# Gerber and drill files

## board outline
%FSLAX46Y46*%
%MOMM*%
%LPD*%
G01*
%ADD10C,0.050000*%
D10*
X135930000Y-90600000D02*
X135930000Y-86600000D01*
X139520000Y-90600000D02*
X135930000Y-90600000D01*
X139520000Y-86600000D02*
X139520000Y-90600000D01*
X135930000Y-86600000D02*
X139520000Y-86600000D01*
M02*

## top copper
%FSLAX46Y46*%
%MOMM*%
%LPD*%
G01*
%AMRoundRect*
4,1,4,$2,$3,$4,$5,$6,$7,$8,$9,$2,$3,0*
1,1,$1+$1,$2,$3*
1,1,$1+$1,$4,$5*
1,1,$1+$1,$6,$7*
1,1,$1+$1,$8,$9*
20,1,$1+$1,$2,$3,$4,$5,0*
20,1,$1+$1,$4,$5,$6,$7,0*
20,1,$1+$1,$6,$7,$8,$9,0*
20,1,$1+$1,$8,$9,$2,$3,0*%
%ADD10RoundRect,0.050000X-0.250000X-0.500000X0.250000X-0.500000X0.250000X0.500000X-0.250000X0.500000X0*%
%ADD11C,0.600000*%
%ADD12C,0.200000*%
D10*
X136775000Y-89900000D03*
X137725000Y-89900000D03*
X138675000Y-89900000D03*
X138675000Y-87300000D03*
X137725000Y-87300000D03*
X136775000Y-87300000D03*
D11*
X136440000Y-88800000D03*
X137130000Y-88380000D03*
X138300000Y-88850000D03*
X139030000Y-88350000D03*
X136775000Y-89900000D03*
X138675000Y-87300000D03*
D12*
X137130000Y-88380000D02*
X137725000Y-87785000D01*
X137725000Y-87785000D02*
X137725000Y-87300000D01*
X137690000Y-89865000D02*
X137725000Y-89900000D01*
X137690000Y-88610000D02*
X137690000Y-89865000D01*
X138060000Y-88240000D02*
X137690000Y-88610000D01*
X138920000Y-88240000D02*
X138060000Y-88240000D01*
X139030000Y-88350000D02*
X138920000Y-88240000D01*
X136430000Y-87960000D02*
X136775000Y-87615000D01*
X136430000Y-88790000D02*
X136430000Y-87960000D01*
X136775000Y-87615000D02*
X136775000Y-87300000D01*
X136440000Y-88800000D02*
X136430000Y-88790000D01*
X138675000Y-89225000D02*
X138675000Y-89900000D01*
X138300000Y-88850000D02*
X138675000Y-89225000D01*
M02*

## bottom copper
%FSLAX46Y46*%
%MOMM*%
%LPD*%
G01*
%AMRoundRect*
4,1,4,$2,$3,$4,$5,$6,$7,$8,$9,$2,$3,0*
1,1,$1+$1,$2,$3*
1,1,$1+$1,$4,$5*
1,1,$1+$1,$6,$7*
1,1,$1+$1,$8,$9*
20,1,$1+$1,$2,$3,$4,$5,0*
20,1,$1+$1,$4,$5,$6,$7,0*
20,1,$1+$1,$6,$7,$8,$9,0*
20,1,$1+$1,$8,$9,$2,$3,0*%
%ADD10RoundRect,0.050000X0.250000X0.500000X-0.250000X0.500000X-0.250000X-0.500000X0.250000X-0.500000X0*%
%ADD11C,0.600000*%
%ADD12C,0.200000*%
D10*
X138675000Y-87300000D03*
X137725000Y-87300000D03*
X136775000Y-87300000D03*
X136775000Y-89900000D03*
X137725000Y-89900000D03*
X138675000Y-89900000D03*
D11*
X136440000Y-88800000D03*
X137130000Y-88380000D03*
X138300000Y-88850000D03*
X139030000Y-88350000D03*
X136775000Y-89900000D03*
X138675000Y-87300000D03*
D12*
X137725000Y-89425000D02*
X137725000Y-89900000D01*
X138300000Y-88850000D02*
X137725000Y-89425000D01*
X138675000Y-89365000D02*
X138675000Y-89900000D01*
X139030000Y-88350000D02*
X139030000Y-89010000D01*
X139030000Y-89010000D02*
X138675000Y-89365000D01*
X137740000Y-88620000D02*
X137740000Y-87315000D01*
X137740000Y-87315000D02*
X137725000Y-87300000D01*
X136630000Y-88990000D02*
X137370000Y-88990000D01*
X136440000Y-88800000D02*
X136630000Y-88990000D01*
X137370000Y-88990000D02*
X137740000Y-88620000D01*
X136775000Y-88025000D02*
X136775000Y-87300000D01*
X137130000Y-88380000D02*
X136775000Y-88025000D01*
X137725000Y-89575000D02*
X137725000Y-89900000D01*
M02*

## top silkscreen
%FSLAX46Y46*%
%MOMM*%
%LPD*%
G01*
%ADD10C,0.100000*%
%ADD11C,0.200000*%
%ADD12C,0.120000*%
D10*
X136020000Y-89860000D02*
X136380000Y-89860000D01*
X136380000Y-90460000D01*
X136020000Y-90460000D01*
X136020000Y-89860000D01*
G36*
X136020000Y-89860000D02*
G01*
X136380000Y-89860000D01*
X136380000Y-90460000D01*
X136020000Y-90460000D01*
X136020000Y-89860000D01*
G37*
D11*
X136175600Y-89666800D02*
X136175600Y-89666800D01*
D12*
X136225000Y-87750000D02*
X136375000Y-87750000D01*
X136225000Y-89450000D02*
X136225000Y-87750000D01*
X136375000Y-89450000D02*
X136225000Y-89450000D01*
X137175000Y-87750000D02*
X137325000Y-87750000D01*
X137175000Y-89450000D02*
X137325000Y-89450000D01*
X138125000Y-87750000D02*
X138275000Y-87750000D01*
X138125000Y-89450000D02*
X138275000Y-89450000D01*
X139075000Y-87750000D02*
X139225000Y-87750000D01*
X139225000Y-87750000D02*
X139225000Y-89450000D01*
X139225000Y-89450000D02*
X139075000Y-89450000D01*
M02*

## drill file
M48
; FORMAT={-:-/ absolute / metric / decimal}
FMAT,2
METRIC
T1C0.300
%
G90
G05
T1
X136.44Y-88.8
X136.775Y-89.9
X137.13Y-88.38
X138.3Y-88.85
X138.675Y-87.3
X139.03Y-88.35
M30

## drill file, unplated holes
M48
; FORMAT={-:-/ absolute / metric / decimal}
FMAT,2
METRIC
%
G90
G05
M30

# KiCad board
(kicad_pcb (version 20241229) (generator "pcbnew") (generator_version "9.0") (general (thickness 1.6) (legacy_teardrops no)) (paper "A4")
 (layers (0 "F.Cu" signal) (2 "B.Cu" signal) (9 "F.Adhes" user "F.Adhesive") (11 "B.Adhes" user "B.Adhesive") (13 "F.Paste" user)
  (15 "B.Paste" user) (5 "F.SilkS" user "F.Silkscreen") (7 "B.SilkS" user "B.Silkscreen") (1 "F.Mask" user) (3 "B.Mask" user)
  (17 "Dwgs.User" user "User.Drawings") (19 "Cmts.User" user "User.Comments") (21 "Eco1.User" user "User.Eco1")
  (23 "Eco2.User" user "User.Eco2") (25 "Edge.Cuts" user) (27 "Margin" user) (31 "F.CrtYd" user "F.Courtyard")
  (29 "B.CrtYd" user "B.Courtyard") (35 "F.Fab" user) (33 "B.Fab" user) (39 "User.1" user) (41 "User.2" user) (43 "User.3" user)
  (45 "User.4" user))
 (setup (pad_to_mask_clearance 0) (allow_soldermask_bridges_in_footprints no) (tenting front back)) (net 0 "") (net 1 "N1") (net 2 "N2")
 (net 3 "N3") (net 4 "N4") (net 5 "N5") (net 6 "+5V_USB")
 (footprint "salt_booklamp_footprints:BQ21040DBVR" (layer "F.Cu") (at 137.725 88.6)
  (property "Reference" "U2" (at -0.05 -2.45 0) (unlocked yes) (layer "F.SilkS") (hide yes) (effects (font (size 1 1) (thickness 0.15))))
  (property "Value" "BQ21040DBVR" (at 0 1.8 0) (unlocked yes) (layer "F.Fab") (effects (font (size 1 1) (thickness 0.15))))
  (fp_line (start -1.5494 1.0668) (end -1.5494 1.0668) (stroke (width 0.2) (type default)) (layer "F.SilkS"))
  (fp_line (start -1.5 -0.85) (end -1.35 -0.85) (stroke (width 0.12) (type default)) (layer "F.SilkS"))
  (fp_line (start -1.5 0.85) (end -1.5 -0.85) (stroke (width 0.12) (type default)) (layer "F.SilkS"))
  (fp_line (start -1.35 0.85) (end -1.5 0.85) (stroke (width 0.12) (type default)) (layer "F.SilkS"))
  (fp_line (start -0.55 -0.85) (end -0.4 -0.85) (stroke (width 0.12) (type default)) (layer "F.SilkS"))
  (fp_line (start -0.55 0.85) (end -0.4 0.85) (stroke (width 0.12) (type default)) (layer "F.SilkS"))
  (fp_line (start 0.4 -0.85) (end 0.55 -0.85) (stroke (width 0.12) (type default)) (layer "F.SilkS"))
  (fp_line (start 0.4 0.85) (end 0.55 0.85) (stroke (width 0.12) (type default)) (layer "F.SilkS"))
  (fp_line (start 1.35 -0.85) (end 1.5 -0.85) (stroke (width 0.12) (type default)) (layer "F.SilkS"))
  (fp_line (start 1.5 -0.85) (end 1.5 0.85) (stroke (width 0.12) (type default)) (layer "F.SilkS"))
  (fp_line (start 1.5 0.85) (end 1.35 0.85) (stroke (width 0.12) (type default)) (layer "F.SilkS"))
  (pad "1" smd roundrect (at -0.95 1.3) (size 0.6 1.1) (layers "F.Cu" "F.Mask" "F.Paste") (roundrect_rratio 0.08333333333) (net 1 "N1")
   (thermal_bridge_angle 45))
  (pad "2" smd roundrect (at 0 1.3) (size 0.6 1.1) (layers "F.Cu" "F.Mask" "F.Paste") (roundrect_rratio 0.08333333333) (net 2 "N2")
   (thermal_bridge_angle 45))
  (pad "3" smd roundrect (at 0.95 1.3) (size 0.6 1.1) (layers "F.Cu" "F.Mask" "F.Paste") (roundrect_rratio 0.08333333333) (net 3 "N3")
   (thermal_bridge_angle 45))
  (pad "4" smd roundrect (at 0.95 -1.3) (size 0.6 1.1) (layers "F.Cu" "F.Mask" "F.Paste") (roundrect_rratio 0.08333333333) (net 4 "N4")
   (thermal_bridge_angle 45))
  (pad "5" smd roundrect (at 0 -1.3) (size 0.6 1.1) (layers "F.Cu" "F.Mask" "F.Paste") (roundrect_rratio 0.08333333333) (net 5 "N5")
   (thermal_bridge_angle 45))
  (pad "6" smd roundrect (at -0.95 -1.3) (size 0.6 1.1) (layers "F.Cu" "F.Mask" "F.Paste") (roundrect_rratio 0.08333333333)
   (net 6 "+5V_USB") (thermal_bridge_angle 45)))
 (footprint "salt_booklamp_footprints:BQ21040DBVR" (layer "B.Cu") (at 137.725 88.6 180)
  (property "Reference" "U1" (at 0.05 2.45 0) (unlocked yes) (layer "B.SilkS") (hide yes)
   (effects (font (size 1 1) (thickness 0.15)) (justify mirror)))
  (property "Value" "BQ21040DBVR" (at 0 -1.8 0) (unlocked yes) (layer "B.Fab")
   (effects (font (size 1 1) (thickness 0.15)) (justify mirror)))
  (pad "1" smd roundrect (at -0.95 1.3 180) (size 0.6 1.1) (layers "B.Cu" "B.Mask" "B.Paste") (roundrect_rratio 0.08333333333) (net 4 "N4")
   (thermal_bridge_angle 45))
  (pad "2" smd roundrect (at 0 1.3 180) (size 0.6 1.1) (layers "B.Cu" "B.Mask" "B.Paste") (roundrect_rratio 0.08333333333) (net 6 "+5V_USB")
   (thermal_bridge_angle 45))
  (pad "3" smd roundrect (at 0.95 1.3 180) (size 0.6 1.1) (layers "B.Cu" "B.Mask" "B.Paste") (roundrect_rratio 0.08333333333) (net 5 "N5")
   (thermal_bridge_angle 45))
  (pad "4" smd roundrect (at 0.95 -1.3 180) (size 0.6 1.1) (layers "B.Cu" "B.Mask" "B.Paste") (roundrect_rratio 0.08333333333) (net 1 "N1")
   (thermal_bridge_angle 45))
  (pad "5" smd roundrect (at 0 -1.3 180) (size 0.6 1.1) (layers "B.Cu" "B.Mask" "B.Paste") (roundrect_rratio 0.08333333333) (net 3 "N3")
   (thermal_bridge_angle 45))
  (pad "6" smd roundrect (at -0.95 -1.3 180) (size 0.6 1.1) (layers "B.Cu" "B.Mask" "B.Paste") (roundrect_rratio 0.08333333333) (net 2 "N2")
   (thermal_bridge_angle 45)))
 (gr_rect (start 136.02 89.86) (end 136.38 90.46) (stroke (width 0.1) (type solid)) (fill yes) (layer "F.SilkS"))
 (gr_line (start 135.93 86.6) (end 139.52 86.6) (stroke (width 0.05) (type default)) (layer "Edge.Cuts"))
 (gr_line (start 135.93 90.6) (end 135.93 86.6) (stroke (width 0.05) (type default)) (layer "Edge.Cuts"))
 (gr_line (start 139.52 90.6) (end 135.93 90.6) (stroke (width 0.05) (type default)) (layer "Edge.Cuts"))
 (gr_line (start 139.52 86.6) (end 139.52 90.6) (stroke (width 0.05) (type default)) (layer "Edge.Cuts"))
 (segment (start 136.43 87.96) (end 136.775 87.615) (width 0.2) (layer "F.Cu") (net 6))
 (segment (start 136.43 88.79) (end 136.43 87.96) (width 0.2) (layer "F.Cu") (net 6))
 (segment (start 136.44 88.8) (end 136.43 88.79) (width 0.2) (layer "F.Cu") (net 6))
 (segment (start 136.775 87.615) (end 136.775 87.3) (width 0.2) (layer "F.Cu") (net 6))
 (via (at 136.44 88.8) (size 0.6) (drill 0.3) (layers "F.Cu" "B.Cu") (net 6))
 (segment (start 137.37 88.99) (end 137.74 88.62) (width 0.2) (layer "B.Cu") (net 6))
 (segment (start 136.44 88.8) (end 136.63 88.99) (width 0.2) (layer "B.Cu") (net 6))
 (segment (start 137.74 88.62) (end 137.74 87.315) (width 0.2) (layer "B.Cu") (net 6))
 (segment (start 136.63 88.99) (end 137.37 88.99) (width 0.2) (layer "B.Cu") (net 6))
 (segment (start 137.74 87.315) (end 137.725 87.3) (width 0.2) (layer "B.Cu") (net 6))
 (segment (start 137.69 88.61) (end 137.69 89.865) (width 0.2) (layer "F.Cu") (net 2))
 (segment (start 137.69 89.865) (end 137.725 89.9) (width 0.2) (layer "F.Cu") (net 2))
 (segment (start 138.06 88.24) (end 137.69 88.61) (width 0.2) (layer "F.Cu") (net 2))
 (segment (start 139.03 88.35) (end 138.92 88.24) (width 0.2) (layer "F.Cu") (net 2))
 (segment (start 138.92 88.24) (end 138.06 88.24) (width 0.2) (layer "F.Cu") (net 2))
 (via (at 139.03 88.35) (size 0.6) (drill 0.3) (layers "F.Cu" "B.Cu") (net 2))
 (segment (start 138.675 89.365) (end 138.675 89.9) (width 0.2) (layer "B.Cu") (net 2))
 (segment (start 139.03 88.35) (end 139.03 89.01) (width 0.2) (layer "B.Cu") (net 2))
 (segment (start 139.03 89.01) (end 138.675 89.365) (width 0.2) (layer "B.Cu") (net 2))
 (via (at 138.675 87.3) (size 0.6) (drill 0.3) (layers "F.Cu" "B.Cu") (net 4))
 (segment (start 138.3 88.85) (end 138.675 89.225) (width 0.2) (layer "F.Cu") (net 3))
 (segment (start 138.675 89.225) (end 138.675 89.9) (width 0.2) (layer "F.Cu") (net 3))
 (via (at 138.3 88.85) (size 0.6) (drill 0.3) (layers "F.Cu" "B.Cu") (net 3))
 (segment (start 137.725 89.425) (end 137.725 89.9) (width 0.2) (layer "B.Cu") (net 3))
 (segment (start 138.3 88.85) (end 137.725 89.425) (width 0.2) (layer "B.Cu") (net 3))
 (segment (start 137.725 89.575) (end 137.725 89.9) (width 0.2) (layer "B.Cu") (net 3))
 (segment (start 137.725 87.785) (end 137.725 87.3) (width 0.2) (layer "F.Cu") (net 5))
 (segment (start 137.13 88.38) (end 137.725 87.785) (width 0.2) (layer "F.Cu") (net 5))
 (via (at 137.13 88.38) (size 0.6) (drill 0.3) (layers "F.Cu" "B.Cu") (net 5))
 (segment (start 137.13 88.38) (end 136.775 88.025) (width 0.2) (layer "B.Cu") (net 5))
 (segment (start 136.775 88.025) (end 136.775 87.3) (width 0.2) (layer "B.Cu") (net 5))
 (via (at 136.775 89.9) (size 0.6) (drill 0.3) (layers "F.Cu" "B.Cu") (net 1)))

